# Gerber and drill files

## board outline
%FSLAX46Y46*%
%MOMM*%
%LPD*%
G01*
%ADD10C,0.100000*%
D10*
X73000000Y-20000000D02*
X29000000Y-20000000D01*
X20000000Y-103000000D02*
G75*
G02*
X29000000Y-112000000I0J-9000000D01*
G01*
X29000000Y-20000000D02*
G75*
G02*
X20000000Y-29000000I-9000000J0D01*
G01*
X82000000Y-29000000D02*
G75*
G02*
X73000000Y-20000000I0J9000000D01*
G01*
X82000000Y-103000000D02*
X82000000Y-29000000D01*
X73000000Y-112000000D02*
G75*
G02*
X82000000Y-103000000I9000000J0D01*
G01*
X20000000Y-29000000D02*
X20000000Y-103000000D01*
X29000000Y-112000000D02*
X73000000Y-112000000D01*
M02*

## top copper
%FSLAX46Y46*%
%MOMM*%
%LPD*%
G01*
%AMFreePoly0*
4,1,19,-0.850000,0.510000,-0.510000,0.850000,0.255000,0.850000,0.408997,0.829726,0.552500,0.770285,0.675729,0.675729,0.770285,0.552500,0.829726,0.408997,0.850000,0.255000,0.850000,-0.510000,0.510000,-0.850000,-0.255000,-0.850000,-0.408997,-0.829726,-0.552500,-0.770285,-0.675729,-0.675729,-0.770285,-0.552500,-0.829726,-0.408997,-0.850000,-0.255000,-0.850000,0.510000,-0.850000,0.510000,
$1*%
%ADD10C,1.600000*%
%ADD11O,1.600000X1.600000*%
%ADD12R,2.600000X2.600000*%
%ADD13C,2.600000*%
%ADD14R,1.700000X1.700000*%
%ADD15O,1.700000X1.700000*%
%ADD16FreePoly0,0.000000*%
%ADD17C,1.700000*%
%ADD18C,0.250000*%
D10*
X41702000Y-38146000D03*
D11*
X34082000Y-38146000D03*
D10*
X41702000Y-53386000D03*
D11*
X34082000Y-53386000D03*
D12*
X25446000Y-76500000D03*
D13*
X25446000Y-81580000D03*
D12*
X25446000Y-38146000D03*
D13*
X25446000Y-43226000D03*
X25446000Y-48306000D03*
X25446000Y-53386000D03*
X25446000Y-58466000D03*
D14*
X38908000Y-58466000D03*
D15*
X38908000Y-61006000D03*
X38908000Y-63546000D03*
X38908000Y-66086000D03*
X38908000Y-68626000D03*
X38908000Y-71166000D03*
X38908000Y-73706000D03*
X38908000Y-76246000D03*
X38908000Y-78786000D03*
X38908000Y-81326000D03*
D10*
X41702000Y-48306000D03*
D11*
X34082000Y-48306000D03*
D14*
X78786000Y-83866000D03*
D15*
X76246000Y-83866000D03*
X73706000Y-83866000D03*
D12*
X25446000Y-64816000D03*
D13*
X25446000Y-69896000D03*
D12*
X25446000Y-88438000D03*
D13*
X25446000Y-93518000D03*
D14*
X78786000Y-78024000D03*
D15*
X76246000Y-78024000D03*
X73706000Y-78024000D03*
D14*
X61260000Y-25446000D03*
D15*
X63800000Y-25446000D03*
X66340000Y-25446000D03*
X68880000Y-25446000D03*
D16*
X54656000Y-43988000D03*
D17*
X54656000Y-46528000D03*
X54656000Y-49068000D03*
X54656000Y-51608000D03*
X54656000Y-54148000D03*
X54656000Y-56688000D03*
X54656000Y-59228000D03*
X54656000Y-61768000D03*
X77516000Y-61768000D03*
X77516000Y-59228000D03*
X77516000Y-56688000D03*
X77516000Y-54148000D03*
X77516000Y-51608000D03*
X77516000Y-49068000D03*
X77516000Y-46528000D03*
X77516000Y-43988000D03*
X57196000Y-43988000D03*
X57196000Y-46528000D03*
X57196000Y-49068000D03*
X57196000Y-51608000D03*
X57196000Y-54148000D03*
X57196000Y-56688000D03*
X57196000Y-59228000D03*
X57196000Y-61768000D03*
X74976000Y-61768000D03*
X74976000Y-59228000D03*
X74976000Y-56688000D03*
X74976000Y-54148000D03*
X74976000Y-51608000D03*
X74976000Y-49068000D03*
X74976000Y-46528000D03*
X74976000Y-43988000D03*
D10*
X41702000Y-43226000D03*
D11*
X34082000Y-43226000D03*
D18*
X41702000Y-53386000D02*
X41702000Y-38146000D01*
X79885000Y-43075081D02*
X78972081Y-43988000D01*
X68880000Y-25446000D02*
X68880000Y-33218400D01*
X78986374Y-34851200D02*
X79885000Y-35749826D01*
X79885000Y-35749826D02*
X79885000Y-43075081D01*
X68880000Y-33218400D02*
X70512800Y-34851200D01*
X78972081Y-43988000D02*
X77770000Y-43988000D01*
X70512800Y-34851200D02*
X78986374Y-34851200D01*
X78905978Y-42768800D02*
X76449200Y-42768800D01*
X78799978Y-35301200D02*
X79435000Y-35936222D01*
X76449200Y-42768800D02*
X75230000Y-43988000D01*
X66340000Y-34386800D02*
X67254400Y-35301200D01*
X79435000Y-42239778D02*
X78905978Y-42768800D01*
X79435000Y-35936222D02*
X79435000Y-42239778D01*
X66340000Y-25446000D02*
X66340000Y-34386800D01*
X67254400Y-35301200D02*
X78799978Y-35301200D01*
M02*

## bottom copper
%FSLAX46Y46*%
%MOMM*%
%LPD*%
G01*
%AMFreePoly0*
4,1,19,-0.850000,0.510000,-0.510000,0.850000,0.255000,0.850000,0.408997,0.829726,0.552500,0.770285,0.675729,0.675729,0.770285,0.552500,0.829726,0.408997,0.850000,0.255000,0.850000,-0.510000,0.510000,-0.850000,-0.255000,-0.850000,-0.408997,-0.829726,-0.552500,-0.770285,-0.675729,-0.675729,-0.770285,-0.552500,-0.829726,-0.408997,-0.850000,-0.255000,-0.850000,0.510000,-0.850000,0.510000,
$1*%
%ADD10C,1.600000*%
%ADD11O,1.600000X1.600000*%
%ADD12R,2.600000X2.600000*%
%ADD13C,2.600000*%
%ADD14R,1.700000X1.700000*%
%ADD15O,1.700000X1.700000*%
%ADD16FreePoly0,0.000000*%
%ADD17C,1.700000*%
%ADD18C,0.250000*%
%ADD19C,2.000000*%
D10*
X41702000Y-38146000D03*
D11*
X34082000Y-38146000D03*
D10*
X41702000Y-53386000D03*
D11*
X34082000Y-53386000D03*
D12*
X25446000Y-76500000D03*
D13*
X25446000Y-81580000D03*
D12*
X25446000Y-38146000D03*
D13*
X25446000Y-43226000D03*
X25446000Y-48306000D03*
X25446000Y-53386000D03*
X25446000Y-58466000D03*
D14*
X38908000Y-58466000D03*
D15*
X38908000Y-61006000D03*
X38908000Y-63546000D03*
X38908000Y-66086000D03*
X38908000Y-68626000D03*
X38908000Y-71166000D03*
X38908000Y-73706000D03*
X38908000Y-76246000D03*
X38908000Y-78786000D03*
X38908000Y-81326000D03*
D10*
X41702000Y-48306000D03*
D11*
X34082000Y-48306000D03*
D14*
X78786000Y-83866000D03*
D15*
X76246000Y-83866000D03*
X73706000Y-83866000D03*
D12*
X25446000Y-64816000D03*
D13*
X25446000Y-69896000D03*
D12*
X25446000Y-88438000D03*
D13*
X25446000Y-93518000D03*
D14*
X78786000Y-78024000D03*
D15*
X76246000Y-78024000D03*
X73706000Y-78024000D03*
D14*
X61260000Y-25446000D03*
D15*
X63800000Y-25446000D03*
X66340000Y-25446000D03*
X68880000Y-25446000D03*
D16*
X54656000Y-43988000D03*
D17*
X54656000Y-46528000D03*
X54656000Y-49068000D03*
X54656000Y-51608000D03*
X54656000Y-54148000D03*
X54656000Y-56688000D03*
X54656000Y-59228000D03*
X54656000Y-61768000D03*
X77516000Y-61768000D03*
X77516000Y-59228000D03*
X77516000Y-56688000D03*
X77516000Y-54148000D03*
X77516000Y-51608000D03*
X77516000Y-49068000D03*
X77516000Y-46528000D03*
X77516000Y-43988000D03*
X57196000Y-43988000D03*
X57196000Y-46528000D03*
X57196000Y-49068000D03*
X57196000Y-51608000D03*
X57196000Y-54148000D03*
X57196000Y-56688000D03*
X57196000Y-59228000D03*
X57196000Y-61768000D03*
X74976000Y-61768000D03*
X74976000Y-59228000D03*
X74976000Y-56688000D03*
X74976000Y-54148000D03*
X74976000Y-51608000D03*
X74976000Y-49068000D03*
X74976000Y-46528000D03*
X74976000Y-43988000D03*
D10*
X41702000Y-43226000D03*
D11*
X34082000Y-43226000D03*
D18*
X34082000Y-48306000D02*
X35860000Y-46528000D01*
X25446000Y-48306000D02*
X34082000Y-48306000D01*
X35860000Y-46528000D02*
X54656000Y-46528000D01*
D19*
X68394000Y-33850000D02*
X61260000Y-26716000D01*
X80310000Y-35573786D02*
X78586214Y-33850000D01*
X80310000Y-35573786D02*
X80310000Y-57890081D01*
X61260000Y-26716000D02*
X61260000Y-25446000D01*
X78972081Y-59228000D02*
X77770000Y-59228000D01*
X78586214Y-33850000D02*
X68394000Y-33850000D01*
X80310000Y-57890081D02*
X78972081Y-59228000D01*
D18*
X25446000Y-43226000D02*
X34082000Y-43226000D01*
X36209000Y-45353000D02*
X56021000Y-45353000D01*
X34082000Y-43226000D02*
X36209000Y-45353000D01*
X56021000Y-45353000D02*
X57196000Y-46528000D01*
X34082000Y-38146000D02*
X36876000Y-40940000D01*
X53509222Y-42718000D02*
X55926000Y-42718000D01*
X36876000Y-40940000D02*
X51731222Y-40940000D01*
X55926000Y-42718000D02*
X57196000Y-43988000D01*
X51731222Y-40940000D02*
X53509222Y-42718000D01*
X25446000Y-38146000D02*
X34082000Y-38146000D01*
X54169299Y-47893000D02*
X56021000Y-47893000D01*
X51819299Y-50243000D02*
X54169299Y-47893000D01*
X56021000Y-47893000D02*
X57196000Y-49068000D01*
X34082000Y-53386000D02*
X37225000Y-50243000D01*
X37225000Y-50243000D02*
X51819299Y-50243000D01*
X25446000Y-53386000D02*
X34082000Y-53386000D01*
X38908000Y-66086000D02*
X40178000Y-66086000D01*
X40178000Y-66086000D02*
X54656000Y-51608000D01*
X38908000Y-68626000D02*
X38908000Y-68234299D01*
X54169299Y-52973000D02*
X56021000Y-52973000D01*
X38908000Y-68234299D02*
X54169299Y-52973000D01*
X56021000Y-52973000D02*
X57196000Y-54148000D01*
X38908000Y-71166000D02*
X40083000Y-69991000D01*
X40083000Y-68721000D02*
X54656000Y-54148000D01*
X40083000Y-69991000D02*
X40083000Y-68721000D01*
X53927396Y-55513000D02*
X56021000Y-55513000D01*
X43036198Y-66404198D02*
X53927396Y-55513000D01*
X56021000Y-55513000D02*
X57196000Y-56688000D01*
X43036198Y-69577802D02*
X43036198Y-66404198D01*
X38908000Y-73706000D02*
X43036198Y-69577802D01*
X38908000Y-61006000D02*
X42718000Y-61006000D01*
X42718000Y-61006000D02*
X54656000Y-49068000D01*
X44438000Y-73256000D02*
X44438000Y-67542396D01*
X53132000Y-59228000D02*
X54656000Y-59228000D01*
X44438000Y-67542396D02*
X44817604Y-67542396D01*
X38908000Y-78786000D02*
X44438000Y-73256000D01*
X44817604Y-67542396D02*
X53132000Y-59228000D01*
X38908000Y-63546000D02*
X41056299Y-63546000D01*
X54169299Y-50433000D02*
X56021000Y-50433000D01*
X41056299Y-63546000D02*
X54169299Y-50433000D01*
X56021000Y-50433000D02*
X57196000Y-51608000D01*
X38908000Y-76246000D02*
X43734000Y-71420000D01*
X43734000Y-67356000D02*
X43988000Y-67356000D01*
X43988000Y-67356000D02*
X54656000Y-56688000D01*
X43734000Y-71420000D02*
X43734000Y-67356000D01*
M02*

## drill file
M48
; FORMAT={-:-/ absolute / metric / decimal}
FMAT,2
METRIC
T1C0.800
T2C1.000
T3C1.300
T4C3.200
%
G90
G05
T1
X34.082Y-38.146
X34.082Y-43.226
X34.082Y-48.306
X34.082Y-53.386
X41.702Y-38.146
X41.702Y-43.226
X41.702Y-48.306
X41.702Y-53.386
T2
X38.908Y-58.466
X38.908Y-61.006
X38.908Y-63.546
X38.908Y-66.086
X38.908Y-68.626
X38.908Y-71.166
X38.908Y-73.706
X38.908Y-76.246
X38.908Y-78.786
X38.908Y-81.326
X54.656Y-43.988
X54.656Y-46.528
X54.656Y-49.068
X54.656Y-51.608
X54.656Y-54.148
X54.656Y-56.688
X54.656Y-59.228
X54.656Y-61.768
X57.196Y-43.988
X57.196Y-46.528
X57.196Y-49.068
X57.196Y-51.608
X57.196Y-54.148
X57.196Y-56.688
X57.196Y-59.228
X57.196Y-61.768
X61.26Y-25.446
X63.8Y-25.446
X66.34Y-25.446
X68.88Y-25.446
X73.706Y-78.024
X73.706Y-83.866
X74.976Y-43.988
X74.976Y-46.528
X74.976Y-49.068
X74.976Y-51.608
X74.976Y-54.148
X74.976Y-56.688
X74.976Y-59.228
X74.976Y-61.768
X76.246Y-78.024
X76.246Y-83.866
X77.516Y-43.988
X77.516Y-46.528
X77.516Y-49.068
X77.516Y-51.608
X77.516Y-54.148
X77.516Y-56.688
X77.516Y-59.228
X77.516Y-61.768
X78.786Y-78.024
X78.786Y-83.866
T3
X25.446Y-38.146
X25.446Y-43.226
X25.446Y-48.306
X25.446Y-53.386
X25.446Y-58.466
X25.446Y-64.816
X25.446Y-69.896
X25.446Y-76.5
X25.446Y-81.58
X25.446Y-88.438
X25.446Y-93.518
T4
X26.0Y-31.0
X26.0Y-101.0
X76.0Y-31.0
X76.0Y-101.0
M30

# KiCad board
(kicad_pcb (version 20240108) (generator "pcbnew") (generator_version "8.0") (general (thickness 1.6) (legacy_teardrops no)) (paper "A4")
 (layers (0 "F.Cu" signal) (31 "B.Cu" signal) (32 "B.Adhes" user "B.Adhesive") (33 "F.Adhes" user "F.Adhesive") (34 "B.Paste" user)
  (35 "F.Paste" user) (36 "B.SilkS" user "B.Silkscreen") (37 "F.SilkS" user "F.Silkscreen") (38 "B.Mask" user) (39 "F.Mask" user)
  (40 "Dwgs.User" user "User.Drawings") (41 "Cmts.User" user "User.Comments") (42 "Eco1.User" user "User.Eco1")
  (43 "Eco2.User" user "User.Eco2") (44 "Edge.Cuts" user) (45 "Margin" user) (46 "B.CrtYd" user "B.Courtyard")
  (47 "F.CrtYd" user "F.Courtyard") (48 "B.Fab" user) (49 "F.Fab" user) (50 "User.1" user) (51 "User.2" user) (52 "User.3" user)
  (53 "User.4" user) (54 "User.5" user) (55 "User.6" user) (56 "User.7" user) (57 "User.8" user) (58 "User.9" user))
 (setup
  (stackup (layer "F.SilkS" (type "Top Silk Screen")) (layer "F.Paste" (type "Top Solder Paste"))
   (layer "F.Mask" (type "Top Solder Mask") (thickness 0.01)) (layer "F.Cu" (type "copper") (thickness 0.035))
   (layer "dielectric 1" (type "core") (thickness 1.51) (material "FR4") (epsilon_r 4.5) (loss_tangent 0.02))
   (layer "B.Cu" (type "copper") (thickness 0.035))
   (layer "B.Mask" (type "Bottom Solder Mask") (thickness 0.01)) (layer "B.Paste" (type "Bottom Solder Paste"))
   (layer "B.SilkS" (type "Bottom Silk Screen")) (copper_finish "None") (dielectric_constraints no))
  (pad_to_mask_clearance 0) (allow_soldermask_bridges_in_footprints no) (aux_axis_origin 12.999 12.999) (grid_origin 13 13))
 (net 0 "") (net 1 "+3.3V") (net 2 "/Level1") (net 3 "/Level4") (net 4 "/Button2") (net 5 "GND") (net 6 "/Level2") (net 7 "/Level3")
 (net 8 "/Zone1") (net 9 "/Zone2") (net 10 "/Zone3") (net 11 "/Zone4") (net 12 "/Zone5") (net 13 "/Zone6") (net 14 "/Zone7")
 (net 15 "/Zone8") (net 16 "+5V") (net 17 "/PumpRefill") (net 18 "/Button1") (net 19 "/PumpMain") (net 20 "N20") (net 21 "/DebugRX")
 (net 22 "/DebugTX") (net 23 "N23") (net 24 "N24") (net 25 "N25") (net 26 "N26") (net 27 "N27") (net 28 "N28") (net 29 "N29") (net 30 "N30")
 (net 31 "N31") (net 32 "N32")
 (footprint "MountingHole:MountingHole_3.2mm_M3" (layer "F.Cu") (at 26 31)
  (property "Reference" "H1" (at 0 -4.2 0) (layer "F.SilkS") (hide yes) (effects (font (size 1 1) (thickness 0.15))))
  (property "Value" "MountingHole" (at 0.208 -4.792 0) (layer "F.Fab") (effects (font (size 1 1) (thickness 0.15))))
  (pad "" np_thru_hole circle (at 0 0) (size 3.2 3.2) (drill 3.2) (layers "*.Cu" "*.Mask")))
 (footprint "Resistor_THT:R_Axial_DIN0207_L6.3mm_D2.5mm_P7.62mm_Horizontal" (layer "F.Cu") (at 41.702 38.146 180)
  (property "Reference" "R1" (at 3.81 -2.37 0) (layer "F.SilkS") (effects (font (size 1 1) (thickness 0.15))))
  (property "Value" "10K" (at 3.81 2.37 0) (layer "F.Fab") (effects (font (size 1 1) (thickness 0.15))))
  (pad "1" thru_hole circle (at 0 0 180) (size 1.6 1.6) (drill 0.8) (layers "*.Cu" "*.Mask") (remove_unused_layers no) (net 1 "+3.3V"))
  (pad "2" thru_hole oval (at 7.62 0 180) (size 1.6 1.6) (drill 0.8) (layers "*.Cu" "*.Mask") (remove_unused_layers no) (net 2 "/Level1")))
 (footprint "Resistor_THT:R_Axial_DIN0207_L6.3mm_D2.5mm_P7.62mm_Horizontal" (layer "F.Cu") (at 41.702 53.386 180)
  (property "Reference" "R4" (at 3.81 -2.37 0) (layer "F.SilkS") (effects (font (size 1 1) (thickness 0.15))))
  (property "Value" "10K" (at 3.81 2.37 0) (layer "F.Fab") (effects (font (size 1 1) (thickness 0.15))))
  (pad "1" thru_hole circle (at 0 0 180) (size 1.6 1.6) (drill 0.8) (layers "*.Cu" "*.Mask") (remove_unused_layers no) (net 1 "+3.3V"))
  (pad "2" thru_hole oval (at 7.62 0 180) (size 1.6 1.6) (drill 0.8) (layers "*.Cu" "*.Mask") (remove_unused_layers no) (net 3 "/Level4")))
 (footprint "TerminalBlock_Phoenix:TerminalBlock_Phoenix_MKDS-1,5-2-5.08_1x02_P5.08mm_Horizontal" (layer "F.Cu") (at 25.446 76.5 -90)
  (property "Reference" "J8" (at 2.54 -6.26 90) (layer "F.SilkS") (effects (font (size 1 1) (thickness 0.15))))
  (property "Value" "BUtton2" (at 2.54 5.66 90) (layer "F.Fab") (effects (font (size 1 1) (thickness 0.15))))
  (pad "1" thru_hole rect (at 0 0 270) (size 2.6 2.6) (drill 1.3) (layers "*.Cu" "*.Mask") (remove_unused_layers no) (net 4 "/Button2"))
  (pad "2" thru_hole circle (at 5.08 0 270) (size 2.6 2.6) (drill 1.3) (layers "*.Cu" "*.Mask") (remove_unused_layers no) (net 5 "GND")))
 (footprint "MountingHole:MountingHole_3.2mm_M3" (layer "F.Cu") (at 26 101)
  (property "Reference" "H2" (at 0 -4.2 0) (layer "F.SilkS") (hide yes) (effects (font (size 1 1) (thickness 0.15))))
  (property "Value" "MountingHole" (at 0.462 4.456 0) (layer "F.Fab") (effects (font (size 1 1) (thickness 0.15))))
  (pad "" np_thru_hole circle (at 0 0) (size 3.2 3.2) (drill 3.2) (layers "*.Cu" "*.Mask")))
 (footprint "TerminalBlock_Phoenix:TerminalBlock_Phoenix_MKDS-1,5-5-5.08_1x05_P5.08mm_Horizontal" (layer "F.Cu") (at 25.446 38.146 -90)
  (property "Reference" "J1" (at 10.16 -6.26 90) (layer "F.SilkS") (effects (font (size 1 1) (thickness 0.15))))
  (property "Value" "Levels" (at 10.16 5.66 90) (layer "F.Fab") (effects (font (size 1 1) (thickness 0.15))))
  (pad "1" thru_hole rect (at 0 0 270) (size 2.6 2.6) (drill 1.3) (layers "*.Cu" "*.Mask") (remove_unused_layers no) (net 2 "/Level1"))
  (pad "2" thru_hole circle (at 5.08 0 270) (size 2.6 2.6) (drill 1.3) (layers "*.Cu" "*.Mask") (remove_unused_layers no) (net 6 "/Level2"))
  (pad "3" thru_hole circle (at 10.16 0 270) (size 2.6 2.6) (drill 1.3) (layers "*.Cu" "*.Mask") (remove_unused_layers no) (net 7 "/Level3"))
  (pad "4" thru_hole circle (at 15.24 0 270) (size 2.6 2.6) (drill 1.3) (layers "*.Cu" "*.Mask") (remove_unused_layers no) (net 3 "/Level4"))
  (pad "5" thru_hole circle (at 20.32 0 270) (size 2.6 2.6) (drill 1.3) (layers "*.Cu" "*.Mask") (remove_unused_layers no) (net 5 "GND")))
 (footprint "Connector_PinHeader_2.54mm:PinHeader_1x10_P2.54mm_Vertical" (layer "F.Cu") (at 38.908 58.466)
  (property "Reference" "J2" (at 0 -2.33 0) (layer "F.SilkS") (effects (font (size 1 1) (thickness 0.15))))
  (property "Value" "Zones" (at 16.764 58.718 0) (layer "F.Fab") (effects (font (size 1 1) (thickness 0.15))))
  (pad "1" thru_hole rect (at 0 0) (size 1.7 1.7) (drill 1) (layers "*.Cu" "*.Mask") (remove_unused_layers no) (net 5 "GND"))
  (pad "2" thru_hole oval (at 0 2.54) (size 1.7 1.7) (drill 1) (layers "*.Cu" "*.Mask") (remove_unused_layers no) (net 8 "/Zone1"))
  (pad "3" thru_hole oval (at 0 5.08) (size 1.7 1.7) (drill 1) (layers "*.Cu" "*.Mask") (remove_unused_layers no) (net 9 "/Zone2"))
  (pad "4" thru_hole oval (at 0 7.62) (size 1.7 1.7) (drill 1) (layers "*.Cu" "*.Mask") (remove_unused_layers no) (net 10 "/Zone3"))
  (pad "5" thru_hole oval (at 0 10.16) (size 1.7 1.7) (drill 1) (layers "*.Cu" "*.Mask") (remove_unused_layers no) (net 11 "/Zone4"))
  (pad "6" thru_hole oval (at 0 12.7) (size 1.7 1.7) (drill 1) (layers "*.Cu" "*.Mask") (remove_unused_layers no) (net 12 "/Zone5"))
  (pad "7" thru_hole oval (at 0 15.24) (size 1.7 1.7) (drill 1) (layers "*.Cu" "*.Mask") (remove_unused_layers no) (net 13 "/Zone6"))
  (pad "8" thru_hole oval (at 0 17.78) (size 1.7 1.7) (drill 1) (layers "*.Cu" "*.Mask") (remove_unused_layers no) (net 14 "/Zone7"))
  (pad "9" thru_hole oval (at 0 20.32) (size 1.7 1.7) (drill 1) (layers "*.Cu" "*.Mask") (remove_unused_layers no) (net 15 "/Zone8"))
  (pad "10" thru_hole oval (at 0 22.86) (size 1.7 1.7) (drill 1) (layers "*.Cu" "*.Mask") (remove_unused_layers no) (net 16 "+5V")))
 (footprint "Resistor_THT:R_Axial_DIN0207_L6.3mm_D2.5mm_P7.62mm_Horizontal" (layer "F.Cu") (at 41.702 48.306 180)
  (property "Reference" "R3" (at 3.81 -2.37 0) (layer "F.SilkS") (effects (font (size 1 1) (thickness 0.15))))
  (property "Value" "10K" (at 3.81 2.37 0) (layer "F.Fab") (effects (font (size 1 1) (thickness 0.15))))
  (pad "1" thru_hole circle (at 0 0 180) (size 1.6 1.6) (drill 0.8) (layers "*.Cu" "*.Mask") (remove_unused_layers no) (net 1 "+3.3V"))
  (pad "2" thru_hole oval (at 7.62 0 180) (size 1.6 1.6) (drill 0.8) (layers "*.Cu" "*.Mask") (remove_unused_layers no) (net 7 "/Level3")))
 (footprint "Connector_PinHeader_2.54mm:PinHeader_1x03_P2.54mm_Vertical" (layer "F.Cu") (at 78.786 83.866 -90)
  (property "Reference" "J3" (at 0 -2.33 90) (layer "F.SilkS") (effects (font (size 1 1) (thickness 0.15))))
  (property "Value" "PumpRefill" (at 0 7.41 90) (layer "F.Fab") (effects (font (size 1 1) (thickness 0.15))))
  (pad "1" thru_hole rect (at 0 0 270) (size 1.7 1.7) (drill 1) (layers "*.Cu" "*.Mask") (remove_unused_layers no) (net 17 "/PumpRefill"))
  (pad "2" thru_hole oval (at 0 2.54 270) (size 1.7 1.7) (drill 1) (layers "*.Cu" "*.Mask") (remove_unused_layers no) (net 16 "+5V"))
  (pad "3" thru_hole oval (at 0 5.08 270) (size 1.7 1.7) (drill 1) (layers "*.Cu" "*.Mask") (remove_unused_layers no) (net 5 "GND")))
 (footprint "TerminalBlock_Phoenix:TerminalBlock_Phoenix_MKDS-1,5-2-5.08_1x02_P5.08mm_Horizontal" (layer "F.Cu") (at 25.446 64.816 -90)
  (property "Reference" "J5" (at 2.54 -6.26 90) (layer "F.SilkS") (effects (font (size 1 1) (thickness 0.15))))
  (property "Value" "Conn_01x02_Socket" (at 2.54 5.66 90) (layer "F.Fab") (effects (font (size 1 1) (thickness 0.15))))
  (pad "1" thru_hole rect (at 0 0 270) (size 2.6 2.6) (drill 1.3) (layers "*.Cu" "*.Mask") (remove_unused_layers no) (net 16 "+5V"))
  (pad "2" thru_hole circle (at 5.08 0 270) (size 2.6 2.6) (drill 1.3) (layers "*.Cu" "*.Mask") (remove_unused_layers no) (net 5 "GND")))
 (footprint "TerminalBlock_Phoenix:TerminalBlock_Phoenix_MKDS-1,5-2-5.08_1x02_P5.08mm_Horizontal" (layer "F.Cu") (at 25.446 88.438 -90)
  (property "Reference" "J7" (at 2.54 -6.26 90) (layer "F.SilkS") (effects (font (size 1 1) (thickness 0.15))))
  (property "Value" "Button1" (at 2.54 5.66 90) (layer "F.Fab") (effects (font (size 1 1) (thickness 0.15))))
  (pad "1" thru_hole rect (at 0 0 270) (size 2.6 2.6) (drill 1.3) (layers "*.Cu" "*.Mask") (remove_unused_layers no) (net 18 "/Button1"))
  (pad "2" thru_hole circle (at 5.08 0 270) (size 2.6 2.6) (drill 1.3) (layers "*.Cu" "*.Mask") (remove_unused_layers no) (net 5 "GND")))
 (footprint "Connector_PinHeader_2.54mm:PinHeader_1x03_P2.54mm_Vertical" (layer "F.Cu") (at 78.786 78.024 -90)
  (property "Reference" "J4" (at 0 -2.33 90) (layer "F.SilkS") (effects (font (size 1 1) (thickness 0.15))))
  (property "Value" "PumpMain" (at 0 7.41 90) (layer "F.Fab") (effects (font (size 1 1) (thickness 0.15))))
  (pad "1" thru_hole rect (at 0 0 270) (size 1.7 1.7) (drill 1) (layers "*.Cu" "*.Mask") (remove_unused_layers no) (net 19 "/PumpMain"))
  (pad "2" thru_hole oval (at 0 2.54 270) (size 1.7 1.7) (drill 1) (layers "*.Cu" "*.Mask") (remove_unused_layers no) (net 16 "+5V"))
  (pad "3" thru_hole oval (at 0 5.08 270) (size 1.7 1.7) (drill 1) (layers "*.Cu" "*.Mask") (remove_unused_layers no) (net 5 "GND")))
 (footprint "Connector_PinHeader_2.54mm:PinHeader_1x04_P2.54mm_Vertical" (layer "F.Cu") (at 61.26 25.446 90)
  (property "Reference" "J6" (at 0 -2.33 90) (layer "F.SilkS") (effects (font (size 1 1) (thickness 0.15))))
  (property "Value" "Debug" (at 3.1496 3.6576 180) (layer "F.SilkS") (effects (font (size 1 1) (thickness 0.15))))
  (pad "1" thru_hole rect (at 0 0 90) (size 1.7 1.7) (drill 1) (layers "*.Cu" "*.Mask") (remove_unused_layers no) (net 5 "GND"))
  (pad "2" thru_hole oval (at 0 2.54 90) (size 1.7 1.7) (drill 1) (layers "*.Cu" "*.Mask") (remove_unused_layers no) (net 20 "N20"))
  (pad "3" thru_hole oval (at 0 5.08 90) (size 1.7 1.7) (drill 1) (layers "*.Cu" "*.Mask") (remove_unused_layers no) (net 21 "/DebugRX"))
  (pad "4" thru_hole oval (at 0 7.62 90) (size 1.7 1.7) (drill 1) (layers "*.Cu" "*.Mask") (remove_unused_layers no) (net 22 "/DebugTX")))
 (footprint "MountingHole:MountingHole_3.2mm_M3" (layer "F.Cu") (at 76 101)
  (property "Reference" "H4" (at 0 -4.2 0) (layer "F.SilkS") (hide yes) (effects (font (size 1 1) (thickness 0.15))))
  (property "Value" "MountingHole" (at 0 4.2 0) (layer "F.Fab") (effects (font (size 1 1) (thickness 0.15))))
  (pad "" np_thru_hole circle (at 0 0) (size 3.2 3.2) (drill 3.2) (layers "*.Cu" "*.Mask")))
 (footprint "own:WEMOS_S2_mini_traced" (layer "F.Cu") (at 54.656 43.988)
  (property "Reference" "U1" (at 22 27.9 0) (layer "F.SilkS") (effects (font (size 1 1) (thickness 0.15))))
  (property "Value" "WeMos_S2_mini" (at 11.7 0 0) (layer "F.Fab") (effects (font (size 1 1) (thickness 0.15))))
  (pad "1" thru_hole roundrect (at 0 0) (size 1.7 1.7) (drill 1) (layers "*.Cu" "*.Mask") (remove_unused_layers no) (roundrect_rratio 0.35)
   (chamfer_ratio 0.2) (chamfer top_left bottom_right) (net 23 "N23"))
  (pad "2" thru_hole circle (at 0 2.54) (size 1.7 1.7) (drill 1) (layers "*.Cu" "*.Mask") (remove_unused_layers no) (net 7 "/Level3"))
  (pad "3" thru_hole circle (at 0 5.08) (size 1.7 1.7) (drill 1) (layers "*.Cu" "*.Mask") (remove_unused_layers no) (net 8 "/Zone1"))
  (pad "4" thru_hole circle (at 0 7.62) (size 1.7 1.7) (drill 1) (layers "*.Cu" "*.Mask") (remove_unused_layers no) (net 10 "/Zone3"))
  (pad "5" thru_hole circle (at 0 10.16) (size 1.7 1.7) (drill 1) (layers "*.Cu" "*.Mask") (remove_unused_layers no) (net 12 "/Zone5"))
  (pad "6" thru_hole circle (at 0 12.7) (size 1.7 1.7) (drill 1) (layers "*.Cu" "*.Mask") (remove_unused_layers no) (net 14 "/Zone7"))
  (pad "7" thru_hole circle (at 0 15.24) (size 1.7 1.7) (drill 1) (layers "*.Cu" "*.Mask") (remove_unused_layers no) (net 15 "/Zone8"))
  (pad "8" thru_hole circle (at 0 17.78) (size 1.7 1.7) (drill 1) (layers "*.Cu" "*.Mask") (remove_unused_layers no) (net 1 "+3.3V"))
  (pad "9" thru_hole circle (at 22.86 17.78) (size 1.7 1.7) (drill 1) (layers "*.Cu" "*.Mask") (remove_unused_layers no) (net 16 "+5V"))
  (pad "10" thru_hole circle (at 22.86 15.24) (size 1.7 1.7) (drill 1) (layers "*.Cu" "*.Mask") (remove_unused_layers no) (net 5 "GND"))
  (pad "11" thru_hole circle (at 22.86 12.7) (size 1.7 1.7) (drill 1) (layers "*.Cu" "*.Mask") (remove_unused_layers no) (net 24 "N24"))
  (pad "12" thru_hole circle (at 22.86 10.16) (size 1.7 1.7) (drill 1) (layers "*.Cu" "*.Mask") (remove_unused_layers no) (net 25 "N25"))
  (pad "13" thru_hole circle (at 22.86 7.62) (size 1.7 1.7) (drill 1) (layers "*.Cu" "*.Mask") (remove_unused_layers no) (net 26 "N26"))
  (pad "14" thru_hole circle (at 22.86 5.08) (size 1.7 1.7) (drill 1) (layers "*.Cu" "*.Mask") (remove_unused_layers no) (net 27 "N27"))
  (pad "15" thru_hole circle (at 22.86 2.54) (size 1.7 1.7) (drill 1) (layers "*.Cu" "*.Mask") (remove_unused_layers no)
   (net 19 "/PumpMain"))
  (pad "16" thru_hole circle (at 22.86 0) (size 1.7 1.7) (drill 1) (layers "*.Cu" "*.Mask") (remove_unused_layers no) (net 22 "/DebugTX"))
  (pad "17" thru_hole circle (at 2.54 0) (size 1.7 1.7) (drill 1) (layers "*.Cu" "*.Mask") (remove_unused_layers no) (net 2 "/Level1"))
  (pad "18" thru_hole circle (at 2.54 2.54) (size 1.7 1.7) (drill 1) (layers "*.Cu" "*.Mask") (remove_unused_layers no) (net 6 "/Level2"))
  (pad "19" thru_hole circle (at 2.54 5.08) (size 1.7 1.7) (drill 1) (layers "*.Cu" "*.Mask") (remove_unused_layers no) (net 3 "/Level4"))
  (pad "20" thru_hole circle (at 2.54 7.62) (size 1.7 1.7) (drill 1) (layers "*.Cu" "*.Mask") (remove_unused_layers no) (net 9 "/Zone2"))
  (pad "21" thru_hole circle (at 2.54 10.16) (size 1.7 1.7) (drill 1) (layers "*.Cu" "*.Mask") (remove_unused_layers no) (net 11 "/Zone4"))
  (pad "22" thru_hole circle (at 2.54 12.7) (size 1.7 1.7) (drill 1) (layers "*.Cu" "*.Mask") (remove_unused_layers no) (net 13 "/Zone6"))
  (pad "23" thru_hole circle (at 2.54 15.24) (size 1.7 1.7) (drill 1) (layers "*.Cu" "*.Mask") (remove_unused_layers no) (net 18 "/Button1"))
  (pad "24" thru_hole circle (at 2.54 17.78) (size 1.7 1.7) (drill 1) (layers "*.Cu" "*.Mask") (remove_unused_layers no) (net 4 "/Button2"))
  (pad "25" thru_hole circle (at 20.32 17.78) (size 1.7 1.7) (drill 1) (layers "*.Cu" "*.Mask") (remove_unused_layers no) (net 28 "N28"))
  (pad "26" thru_hole circle (at 20.32 15.24) (size 1.7 1.7) (drill 1) (layers "*.Cu" "*.Mask") (remove_unused_layers no) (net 5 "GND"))
  (pad "27" thru_hole circle (at 20.32 12.7) (size 1.7 1.7) (drill 1) (layers "*.Cu" "*.Mask") (remove_unused_layers no) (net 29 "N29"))
  (pad "28" thru_hole circle (at 20.32 10.16) (size 1.7 1.7) (drill 1) (layers "*.Cu" "*.Mask") (remove_unused_layers no) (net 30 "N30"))
  (pad "29" thru_hole circle (at 20.32 7.62) (size 1.7 1.7) (drill 1) (layers "*.Cu" "*.Mask") (remove_unused_layers no) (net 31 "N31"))
  (pad "30" thru_hole circle (at 20.32 5.08) (size 1.7 1.7) (drill 1) (layers "*.Cu" "*.Mask") (remove_unused_layers no) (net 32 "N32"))
  (pad "31" thru_hole circle (at 20.32 2.54) (size 1.7 1.7) (drill 1) (layers "*.Cu" "*.Mask") (remove_unused_layers no)
   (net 17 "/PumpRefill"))
  (pad "32" thru_hole circle (at 20.32 0) (size 1.7 1.7) (drill 1) (layers "*.Cu" "*.Mask") (remove_unused_layers no) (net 21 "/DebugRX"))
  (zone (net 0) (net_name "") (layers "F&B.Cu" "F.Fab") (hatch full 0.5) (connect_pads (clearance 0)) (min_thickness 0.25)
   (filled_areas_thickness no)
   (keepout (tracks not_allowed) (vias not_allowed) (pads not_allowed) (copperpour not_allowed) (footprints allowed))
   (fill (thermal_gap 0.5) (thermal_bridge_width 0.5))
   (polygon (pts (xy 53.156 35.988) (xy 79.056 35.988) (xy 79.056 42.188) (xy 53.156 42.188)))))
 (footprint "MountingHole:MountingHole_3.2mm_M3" (layer "F.Cu") (at 76 31)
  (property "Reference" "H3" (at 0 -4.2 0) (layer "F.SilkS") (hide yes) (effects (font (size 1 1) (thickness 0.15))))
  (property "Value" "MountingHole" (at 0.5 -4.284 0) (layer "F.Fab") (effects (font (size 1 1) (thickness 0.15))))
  (pad "" np_thru_hole circle (at 0 0) (size 3.2 3.2) (drill 3.2) (layers "*.Cu" "*.Mask")))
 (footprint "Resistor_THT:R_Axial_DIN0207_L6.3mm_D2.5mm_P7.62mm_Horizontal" (layer "F.Cu") (at 41.702 43.226 180)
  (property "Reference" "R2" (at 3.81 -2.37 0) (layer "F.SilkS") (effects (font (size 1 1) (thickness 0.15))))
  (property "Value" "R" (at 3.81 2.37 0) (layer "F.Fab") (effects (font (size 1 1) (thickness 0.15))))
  (pad "1" thru_hole circle (at 0 0 180) (size 1.6 1.6) (drill 0.8) (layers "*.Cu" "*.Mask") (remove_unused_layers no) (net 1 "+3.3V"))
  (pad "2" thru_hole oval (at 7.62 0 180) (size 1.6 1.6) (drill 0.8) (layers "*.Cu" "*.Mask") (remove_unused_layers no) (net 6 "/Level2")))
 (gr_line (start 73 20) (end 29 20) (stroke (width 0.1) (type default)) (layer "Edge.Cuts"))
 (gr_arc (start 20 103) (mid 26.363961 105.636039) (end 29 112) (stroke (width 0.1) (type default)) (layer "Edge.Cuts"))
 (gr_arc (start 29 20) (mid 26.363961 26.363961) (end 20 29) (stroke (width 0.1) (type default)) (layer "Edge.Cuts"))
 (gr_arc (start 82 29) (mid 75.636039 26.363961) (end 73 20) (stroke (width 0.1) (type default)) (layer "Edge.Cuts"))
 (gr_line (start 82 103) (end 82 29) (stroke (width 0.1) (type default)) (layer "Edge.Cuts"))
 (gr_arc (start 73 112) (mid 75.636039 105.636039) (end 82 103) (stroke (width 0.1) (type default)) (layer "Edge.Cuts"))
 (gr_line (start 20 29) (end 20 103) (stroke (width 0.1) (type default)) (layer "Edge.Cuts"))
 (gr_line (start 29 112) (end 73 112) (stroke (width 0.1) (type default)) (layer "Edge.Cuts"))
 (segment (start 34.082 48.306) (end 35.86 46.528) (width 0.25) (layer "B.Cu") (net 7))
 (segment (start 25.446 48.306) (end 34.082 48.306) (width 0.25) (layer "B.Cu") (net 7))
 (segment (start 35.86 46.528) (end 54.656 46.528) (width 0.25) (layer "B.Cu") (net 7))
 (segment (start 68.394 33.85) (end 61.26 26.716) (width 2) (layer "B.Cu") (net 5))
 (segment (start 80.31 35.573786) (end 78.586214 33.85) (width 2) (layer "B.Cu") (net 5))
 (segment (start 80.31 35.573786) (end 80.31 57.890081) (width 2) (layer "B.Cu") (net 5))
 (segment (start 61.26 26.716) (end 61.26 25.446) (width 2) (layer "B.Cu") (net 5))
 (segment (start 78.972081 59.228) (end 77.77 59.228) (width 2) (layer "B.Cu") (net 5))
 (segment (start 78.586214 33.85) (end 68.394 33.85) (width 2) (layer "B.Cu") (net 5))
 (segment (start 80.31 57.890081) (end 78.972081 59.228) (width 2) (layer "B.Cu") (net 5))
 (segment (start 25.446 43.226) (end 34.082 43.226) (width 0.25) (layer "B.Cu") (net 6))
 (segment (start 36.209 45.353) (end 56.021 45.353) (width 0.25) (layer "B.Cu") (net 6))
 (segment (start 34.082 43.226) (end 36.209 45.353) (width 0.25) (layer "B.Cu") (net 6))
 (segment (start 56.021 45.353) (end 57.196 46.528) (width 0.25) (layer "B.Cu") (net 6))
 (segment (start 34.082 38.146) (end 36.876 40.94) (width 0.25) (layer "B.Cu") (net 2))
 (segment (start 53.509222 42.718) (end 55.926 42.718) (width 0.25) (layer "B.Cu") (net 2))
 (segment (start 36.876 40.94) (end 51.731222 40.94) (width 0.25) (layer "B.Cu") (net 2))
 (segment (start 55.926 42.718) (end 57.196 43.988) (width 0.25) (layer "B.Cu") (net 2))
 (segment (start 51.731222 40.94) (end 53.509222 42.718) (width 0.25) (layer "B.Cu") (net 2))
 (segment (start 25.446 38.146) (end 34.082 38.146) (width 0.25) (layer "B.Cu") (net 2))
 (segment (start 41.702 53.386) (end 41.702 38.146) (width 0.25) (layer "F.Cu") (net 1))
 (segment (start 54.169299 47.893) (end 56.021 47.893) (width 0.25) (layer "B.Cu") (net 3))
 (segment (start 51.819299 50.243) (end 54.169299 47.893) (width 0.25) (layer "B.Cu") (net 3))
 (segment (start 56.021 47.893) (end 57.196 49.068) (width 0.25) (layer "B.Cu") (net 3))
 (segment (start 34.082 53.386) (end 37.225 50.243) (width 0.25) (layer "B.Cu") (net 3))
 (segment (start 37.225 50.243) (end 51.819299 50.243) (width 0.25) (layer "B.Cu") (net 3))
 (segment (start 25.446 53.386) (end 34.082 53.386) (width 0.25) (layer "B.Cu") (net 3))
 (segment (start 38.908 66.086) (end 40.178 66.086) (width 0.25) (layer "B.Cu") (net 10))
 (segment (start 40.178 66.086) (end 54.656 51.608) (width 0.25) (layer "B.Cu") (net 10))
 (segment (start 79.885 43.075081) (end 78.972081 43.988) (width 0.25) (layer "F.Cu") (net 22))
 (segment (start 68.88 25.446) (end 68.88 33.2184) (width 0.25) (layer "F.Cu") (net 22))
 (segment (start 78.986374 34.8512) (end 79.885 35.749826) (width 0.25) (layer "F.Cu") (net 22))
 (segment (start 79.885 35.749826) (end 79.885 43.075081) (width 0.25) (layer "F.Cu") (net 22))
 (segment (start 68.88 33.2184) (end 70.5128 34.8512) (width 0.25) (layer "F.Cu") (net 22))
 (segment (start 78.972081 43.988) (end 77.77 43.988) (width 0.25) (layer "F.Cu") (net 22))
 (segment (start 70.5128 34.8512) (end 78.986374 34.8512) (width 0.25) (layer "F.Cu") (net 22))
 (segment (start 78.905978 42.7688) (end 76.4492 42.7688) (width 0.25) (layer "F.Cu") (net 21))
 (segment (start 78.799978 35.3012) (end 79.435 35.936222) (width 0.25) (layer "F.Cu") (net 21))
 (segment (start 76.4492 42.7688) (end 75.23 43.988) (width 0.25) (layer "F.Cu") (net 21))
 (segment (start 66.34 34.3868) (end 67.2544 35.3012) (width 0.25) (layer "F.Cu") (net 21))
 (segment (start 79.435 42.239778) (end 78.905978 42.7688) (width 0.25) (layer "F.Cu") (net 21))
 (segment (start 79.435 35.936222) (end 79.435 42.239778) (width 0.25) (layer "F.Cu") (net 21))
 (segment (start 66.34 25.446) (end 66.34 34.3868) (width 0.25) (layer "F.Cu") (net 21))
 (segment (start 67.2544 35.3012) (end 78.799978 35.3012) (width 0.25) (layer "F.Cu") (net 21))
 (segment (start 38.908 68.626) (end 38.908 68.234299) (width 0.25) (layer "B.Cu") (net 11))
 (segment (start 54.169299 52.973) (end 56.021 52.973) (width 0.25) (layer "B.Cu") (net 11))
 (segment (start 38.908 68.234299) (end 54.169299 52.973) (width 0.25) (layer "B.Cu") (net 11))
 (segment (start 56.021 52.973) (end 57.196 54.148) (width 0.25) (layer "B.Cu") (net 11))
 (segment (start 38.908 71.166) (end 40.083 69.991) (width 0.25) (layer "B.Cu") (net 12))
 (segment (start 40.083 68.721) (end 54.656 54.148) (width 0.25) (layer "B.Cu") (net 12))
 (segment (start 40.083 69.991) (end 40.083 68.721) (width 0.25) (layer "B.Cu") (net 12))
 (segment (start 53.927396 55.513) (end 56.021 55.513) (width 0.25) (layer "B.Cu") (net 13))
 (segment (start 43.036198 66.404198) (end 53.927396 55.513) (width 0.25) (layer "B.Cu") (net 13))
 (segment (start 56.021 55.513) (end 57.196 56.688) (width 0.25) (layer "B.Cu") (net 13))
 (segment (start 43.036198 69.577802) (end 43.036198 66.404198) (width 0.25) (layer "B.Cu") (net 13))
 (segment (start 38.908 73.706) (end 43.036198 69.577802) (width 0.25) (layer "B.Cu") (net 13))
 (segment (start 38.908 61.006) (end 42.718 61.006) (width 0.25) (layer "B.Cu") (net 8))
 (segment (start 42.718 61.006) (end 54.656 49.068) (width 0.25) (layer "B.Cu") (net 8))
 (segment (start 44.438 73.256) (end 44.438 67.542396) (width 0.25) (layer "B.Cu") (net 15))
 (segment (start 53.132 59.228) (end 54.656 59.228) (width 0.25) (layer "B.Cu") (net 15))
 (segment (start 44.438 67.542396) (end 44.817604 67.542396) (width 0.25) (layer "B.Cu") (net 15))
 (segment (start 38.908 78.786) (end 44.438 73.256) (width 0.25) (layer "B.Cu") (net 15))
 (segment (start 44.817604 67.542396) (end 53.132 59.228) (width 0.25) (layer "B.Cu") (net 15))
 (segment (start 38.908 63.546) (end 41.056299 63.546) (width 0.25) (layer "B.Cu") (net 9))
 (segment (start 54.169299 50.433) (end 56.021 50.433) (width 0.25) (layer "B.Cu") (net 9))
 (segment (start 41.056299 63.546) (end 54.169299 50.433) (width 0.25) (layer "B.Cu") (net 9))
 (segment (start 56.021 50.433) (end 57.196 51.608) (width 0.25) (layer "B.Cu") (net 9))
 (segment (start 38.908 76.246) (end 43.734 71.42) (width 0.25) (layer "B.Cu") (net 14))
 (segment (start 43.734 67.356) (end 43.988 67.356) (width 0.25) (layer "B.Cu") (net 14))
 (segment (start 43.988 67.356) (end 54.656 56.688) (width 0.25) (layer "B.Cu") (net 14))
 (segment (start 43.734 71.42) (end 43.734 67.356) (width 0.25) (layer "B.Cu") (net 14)))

